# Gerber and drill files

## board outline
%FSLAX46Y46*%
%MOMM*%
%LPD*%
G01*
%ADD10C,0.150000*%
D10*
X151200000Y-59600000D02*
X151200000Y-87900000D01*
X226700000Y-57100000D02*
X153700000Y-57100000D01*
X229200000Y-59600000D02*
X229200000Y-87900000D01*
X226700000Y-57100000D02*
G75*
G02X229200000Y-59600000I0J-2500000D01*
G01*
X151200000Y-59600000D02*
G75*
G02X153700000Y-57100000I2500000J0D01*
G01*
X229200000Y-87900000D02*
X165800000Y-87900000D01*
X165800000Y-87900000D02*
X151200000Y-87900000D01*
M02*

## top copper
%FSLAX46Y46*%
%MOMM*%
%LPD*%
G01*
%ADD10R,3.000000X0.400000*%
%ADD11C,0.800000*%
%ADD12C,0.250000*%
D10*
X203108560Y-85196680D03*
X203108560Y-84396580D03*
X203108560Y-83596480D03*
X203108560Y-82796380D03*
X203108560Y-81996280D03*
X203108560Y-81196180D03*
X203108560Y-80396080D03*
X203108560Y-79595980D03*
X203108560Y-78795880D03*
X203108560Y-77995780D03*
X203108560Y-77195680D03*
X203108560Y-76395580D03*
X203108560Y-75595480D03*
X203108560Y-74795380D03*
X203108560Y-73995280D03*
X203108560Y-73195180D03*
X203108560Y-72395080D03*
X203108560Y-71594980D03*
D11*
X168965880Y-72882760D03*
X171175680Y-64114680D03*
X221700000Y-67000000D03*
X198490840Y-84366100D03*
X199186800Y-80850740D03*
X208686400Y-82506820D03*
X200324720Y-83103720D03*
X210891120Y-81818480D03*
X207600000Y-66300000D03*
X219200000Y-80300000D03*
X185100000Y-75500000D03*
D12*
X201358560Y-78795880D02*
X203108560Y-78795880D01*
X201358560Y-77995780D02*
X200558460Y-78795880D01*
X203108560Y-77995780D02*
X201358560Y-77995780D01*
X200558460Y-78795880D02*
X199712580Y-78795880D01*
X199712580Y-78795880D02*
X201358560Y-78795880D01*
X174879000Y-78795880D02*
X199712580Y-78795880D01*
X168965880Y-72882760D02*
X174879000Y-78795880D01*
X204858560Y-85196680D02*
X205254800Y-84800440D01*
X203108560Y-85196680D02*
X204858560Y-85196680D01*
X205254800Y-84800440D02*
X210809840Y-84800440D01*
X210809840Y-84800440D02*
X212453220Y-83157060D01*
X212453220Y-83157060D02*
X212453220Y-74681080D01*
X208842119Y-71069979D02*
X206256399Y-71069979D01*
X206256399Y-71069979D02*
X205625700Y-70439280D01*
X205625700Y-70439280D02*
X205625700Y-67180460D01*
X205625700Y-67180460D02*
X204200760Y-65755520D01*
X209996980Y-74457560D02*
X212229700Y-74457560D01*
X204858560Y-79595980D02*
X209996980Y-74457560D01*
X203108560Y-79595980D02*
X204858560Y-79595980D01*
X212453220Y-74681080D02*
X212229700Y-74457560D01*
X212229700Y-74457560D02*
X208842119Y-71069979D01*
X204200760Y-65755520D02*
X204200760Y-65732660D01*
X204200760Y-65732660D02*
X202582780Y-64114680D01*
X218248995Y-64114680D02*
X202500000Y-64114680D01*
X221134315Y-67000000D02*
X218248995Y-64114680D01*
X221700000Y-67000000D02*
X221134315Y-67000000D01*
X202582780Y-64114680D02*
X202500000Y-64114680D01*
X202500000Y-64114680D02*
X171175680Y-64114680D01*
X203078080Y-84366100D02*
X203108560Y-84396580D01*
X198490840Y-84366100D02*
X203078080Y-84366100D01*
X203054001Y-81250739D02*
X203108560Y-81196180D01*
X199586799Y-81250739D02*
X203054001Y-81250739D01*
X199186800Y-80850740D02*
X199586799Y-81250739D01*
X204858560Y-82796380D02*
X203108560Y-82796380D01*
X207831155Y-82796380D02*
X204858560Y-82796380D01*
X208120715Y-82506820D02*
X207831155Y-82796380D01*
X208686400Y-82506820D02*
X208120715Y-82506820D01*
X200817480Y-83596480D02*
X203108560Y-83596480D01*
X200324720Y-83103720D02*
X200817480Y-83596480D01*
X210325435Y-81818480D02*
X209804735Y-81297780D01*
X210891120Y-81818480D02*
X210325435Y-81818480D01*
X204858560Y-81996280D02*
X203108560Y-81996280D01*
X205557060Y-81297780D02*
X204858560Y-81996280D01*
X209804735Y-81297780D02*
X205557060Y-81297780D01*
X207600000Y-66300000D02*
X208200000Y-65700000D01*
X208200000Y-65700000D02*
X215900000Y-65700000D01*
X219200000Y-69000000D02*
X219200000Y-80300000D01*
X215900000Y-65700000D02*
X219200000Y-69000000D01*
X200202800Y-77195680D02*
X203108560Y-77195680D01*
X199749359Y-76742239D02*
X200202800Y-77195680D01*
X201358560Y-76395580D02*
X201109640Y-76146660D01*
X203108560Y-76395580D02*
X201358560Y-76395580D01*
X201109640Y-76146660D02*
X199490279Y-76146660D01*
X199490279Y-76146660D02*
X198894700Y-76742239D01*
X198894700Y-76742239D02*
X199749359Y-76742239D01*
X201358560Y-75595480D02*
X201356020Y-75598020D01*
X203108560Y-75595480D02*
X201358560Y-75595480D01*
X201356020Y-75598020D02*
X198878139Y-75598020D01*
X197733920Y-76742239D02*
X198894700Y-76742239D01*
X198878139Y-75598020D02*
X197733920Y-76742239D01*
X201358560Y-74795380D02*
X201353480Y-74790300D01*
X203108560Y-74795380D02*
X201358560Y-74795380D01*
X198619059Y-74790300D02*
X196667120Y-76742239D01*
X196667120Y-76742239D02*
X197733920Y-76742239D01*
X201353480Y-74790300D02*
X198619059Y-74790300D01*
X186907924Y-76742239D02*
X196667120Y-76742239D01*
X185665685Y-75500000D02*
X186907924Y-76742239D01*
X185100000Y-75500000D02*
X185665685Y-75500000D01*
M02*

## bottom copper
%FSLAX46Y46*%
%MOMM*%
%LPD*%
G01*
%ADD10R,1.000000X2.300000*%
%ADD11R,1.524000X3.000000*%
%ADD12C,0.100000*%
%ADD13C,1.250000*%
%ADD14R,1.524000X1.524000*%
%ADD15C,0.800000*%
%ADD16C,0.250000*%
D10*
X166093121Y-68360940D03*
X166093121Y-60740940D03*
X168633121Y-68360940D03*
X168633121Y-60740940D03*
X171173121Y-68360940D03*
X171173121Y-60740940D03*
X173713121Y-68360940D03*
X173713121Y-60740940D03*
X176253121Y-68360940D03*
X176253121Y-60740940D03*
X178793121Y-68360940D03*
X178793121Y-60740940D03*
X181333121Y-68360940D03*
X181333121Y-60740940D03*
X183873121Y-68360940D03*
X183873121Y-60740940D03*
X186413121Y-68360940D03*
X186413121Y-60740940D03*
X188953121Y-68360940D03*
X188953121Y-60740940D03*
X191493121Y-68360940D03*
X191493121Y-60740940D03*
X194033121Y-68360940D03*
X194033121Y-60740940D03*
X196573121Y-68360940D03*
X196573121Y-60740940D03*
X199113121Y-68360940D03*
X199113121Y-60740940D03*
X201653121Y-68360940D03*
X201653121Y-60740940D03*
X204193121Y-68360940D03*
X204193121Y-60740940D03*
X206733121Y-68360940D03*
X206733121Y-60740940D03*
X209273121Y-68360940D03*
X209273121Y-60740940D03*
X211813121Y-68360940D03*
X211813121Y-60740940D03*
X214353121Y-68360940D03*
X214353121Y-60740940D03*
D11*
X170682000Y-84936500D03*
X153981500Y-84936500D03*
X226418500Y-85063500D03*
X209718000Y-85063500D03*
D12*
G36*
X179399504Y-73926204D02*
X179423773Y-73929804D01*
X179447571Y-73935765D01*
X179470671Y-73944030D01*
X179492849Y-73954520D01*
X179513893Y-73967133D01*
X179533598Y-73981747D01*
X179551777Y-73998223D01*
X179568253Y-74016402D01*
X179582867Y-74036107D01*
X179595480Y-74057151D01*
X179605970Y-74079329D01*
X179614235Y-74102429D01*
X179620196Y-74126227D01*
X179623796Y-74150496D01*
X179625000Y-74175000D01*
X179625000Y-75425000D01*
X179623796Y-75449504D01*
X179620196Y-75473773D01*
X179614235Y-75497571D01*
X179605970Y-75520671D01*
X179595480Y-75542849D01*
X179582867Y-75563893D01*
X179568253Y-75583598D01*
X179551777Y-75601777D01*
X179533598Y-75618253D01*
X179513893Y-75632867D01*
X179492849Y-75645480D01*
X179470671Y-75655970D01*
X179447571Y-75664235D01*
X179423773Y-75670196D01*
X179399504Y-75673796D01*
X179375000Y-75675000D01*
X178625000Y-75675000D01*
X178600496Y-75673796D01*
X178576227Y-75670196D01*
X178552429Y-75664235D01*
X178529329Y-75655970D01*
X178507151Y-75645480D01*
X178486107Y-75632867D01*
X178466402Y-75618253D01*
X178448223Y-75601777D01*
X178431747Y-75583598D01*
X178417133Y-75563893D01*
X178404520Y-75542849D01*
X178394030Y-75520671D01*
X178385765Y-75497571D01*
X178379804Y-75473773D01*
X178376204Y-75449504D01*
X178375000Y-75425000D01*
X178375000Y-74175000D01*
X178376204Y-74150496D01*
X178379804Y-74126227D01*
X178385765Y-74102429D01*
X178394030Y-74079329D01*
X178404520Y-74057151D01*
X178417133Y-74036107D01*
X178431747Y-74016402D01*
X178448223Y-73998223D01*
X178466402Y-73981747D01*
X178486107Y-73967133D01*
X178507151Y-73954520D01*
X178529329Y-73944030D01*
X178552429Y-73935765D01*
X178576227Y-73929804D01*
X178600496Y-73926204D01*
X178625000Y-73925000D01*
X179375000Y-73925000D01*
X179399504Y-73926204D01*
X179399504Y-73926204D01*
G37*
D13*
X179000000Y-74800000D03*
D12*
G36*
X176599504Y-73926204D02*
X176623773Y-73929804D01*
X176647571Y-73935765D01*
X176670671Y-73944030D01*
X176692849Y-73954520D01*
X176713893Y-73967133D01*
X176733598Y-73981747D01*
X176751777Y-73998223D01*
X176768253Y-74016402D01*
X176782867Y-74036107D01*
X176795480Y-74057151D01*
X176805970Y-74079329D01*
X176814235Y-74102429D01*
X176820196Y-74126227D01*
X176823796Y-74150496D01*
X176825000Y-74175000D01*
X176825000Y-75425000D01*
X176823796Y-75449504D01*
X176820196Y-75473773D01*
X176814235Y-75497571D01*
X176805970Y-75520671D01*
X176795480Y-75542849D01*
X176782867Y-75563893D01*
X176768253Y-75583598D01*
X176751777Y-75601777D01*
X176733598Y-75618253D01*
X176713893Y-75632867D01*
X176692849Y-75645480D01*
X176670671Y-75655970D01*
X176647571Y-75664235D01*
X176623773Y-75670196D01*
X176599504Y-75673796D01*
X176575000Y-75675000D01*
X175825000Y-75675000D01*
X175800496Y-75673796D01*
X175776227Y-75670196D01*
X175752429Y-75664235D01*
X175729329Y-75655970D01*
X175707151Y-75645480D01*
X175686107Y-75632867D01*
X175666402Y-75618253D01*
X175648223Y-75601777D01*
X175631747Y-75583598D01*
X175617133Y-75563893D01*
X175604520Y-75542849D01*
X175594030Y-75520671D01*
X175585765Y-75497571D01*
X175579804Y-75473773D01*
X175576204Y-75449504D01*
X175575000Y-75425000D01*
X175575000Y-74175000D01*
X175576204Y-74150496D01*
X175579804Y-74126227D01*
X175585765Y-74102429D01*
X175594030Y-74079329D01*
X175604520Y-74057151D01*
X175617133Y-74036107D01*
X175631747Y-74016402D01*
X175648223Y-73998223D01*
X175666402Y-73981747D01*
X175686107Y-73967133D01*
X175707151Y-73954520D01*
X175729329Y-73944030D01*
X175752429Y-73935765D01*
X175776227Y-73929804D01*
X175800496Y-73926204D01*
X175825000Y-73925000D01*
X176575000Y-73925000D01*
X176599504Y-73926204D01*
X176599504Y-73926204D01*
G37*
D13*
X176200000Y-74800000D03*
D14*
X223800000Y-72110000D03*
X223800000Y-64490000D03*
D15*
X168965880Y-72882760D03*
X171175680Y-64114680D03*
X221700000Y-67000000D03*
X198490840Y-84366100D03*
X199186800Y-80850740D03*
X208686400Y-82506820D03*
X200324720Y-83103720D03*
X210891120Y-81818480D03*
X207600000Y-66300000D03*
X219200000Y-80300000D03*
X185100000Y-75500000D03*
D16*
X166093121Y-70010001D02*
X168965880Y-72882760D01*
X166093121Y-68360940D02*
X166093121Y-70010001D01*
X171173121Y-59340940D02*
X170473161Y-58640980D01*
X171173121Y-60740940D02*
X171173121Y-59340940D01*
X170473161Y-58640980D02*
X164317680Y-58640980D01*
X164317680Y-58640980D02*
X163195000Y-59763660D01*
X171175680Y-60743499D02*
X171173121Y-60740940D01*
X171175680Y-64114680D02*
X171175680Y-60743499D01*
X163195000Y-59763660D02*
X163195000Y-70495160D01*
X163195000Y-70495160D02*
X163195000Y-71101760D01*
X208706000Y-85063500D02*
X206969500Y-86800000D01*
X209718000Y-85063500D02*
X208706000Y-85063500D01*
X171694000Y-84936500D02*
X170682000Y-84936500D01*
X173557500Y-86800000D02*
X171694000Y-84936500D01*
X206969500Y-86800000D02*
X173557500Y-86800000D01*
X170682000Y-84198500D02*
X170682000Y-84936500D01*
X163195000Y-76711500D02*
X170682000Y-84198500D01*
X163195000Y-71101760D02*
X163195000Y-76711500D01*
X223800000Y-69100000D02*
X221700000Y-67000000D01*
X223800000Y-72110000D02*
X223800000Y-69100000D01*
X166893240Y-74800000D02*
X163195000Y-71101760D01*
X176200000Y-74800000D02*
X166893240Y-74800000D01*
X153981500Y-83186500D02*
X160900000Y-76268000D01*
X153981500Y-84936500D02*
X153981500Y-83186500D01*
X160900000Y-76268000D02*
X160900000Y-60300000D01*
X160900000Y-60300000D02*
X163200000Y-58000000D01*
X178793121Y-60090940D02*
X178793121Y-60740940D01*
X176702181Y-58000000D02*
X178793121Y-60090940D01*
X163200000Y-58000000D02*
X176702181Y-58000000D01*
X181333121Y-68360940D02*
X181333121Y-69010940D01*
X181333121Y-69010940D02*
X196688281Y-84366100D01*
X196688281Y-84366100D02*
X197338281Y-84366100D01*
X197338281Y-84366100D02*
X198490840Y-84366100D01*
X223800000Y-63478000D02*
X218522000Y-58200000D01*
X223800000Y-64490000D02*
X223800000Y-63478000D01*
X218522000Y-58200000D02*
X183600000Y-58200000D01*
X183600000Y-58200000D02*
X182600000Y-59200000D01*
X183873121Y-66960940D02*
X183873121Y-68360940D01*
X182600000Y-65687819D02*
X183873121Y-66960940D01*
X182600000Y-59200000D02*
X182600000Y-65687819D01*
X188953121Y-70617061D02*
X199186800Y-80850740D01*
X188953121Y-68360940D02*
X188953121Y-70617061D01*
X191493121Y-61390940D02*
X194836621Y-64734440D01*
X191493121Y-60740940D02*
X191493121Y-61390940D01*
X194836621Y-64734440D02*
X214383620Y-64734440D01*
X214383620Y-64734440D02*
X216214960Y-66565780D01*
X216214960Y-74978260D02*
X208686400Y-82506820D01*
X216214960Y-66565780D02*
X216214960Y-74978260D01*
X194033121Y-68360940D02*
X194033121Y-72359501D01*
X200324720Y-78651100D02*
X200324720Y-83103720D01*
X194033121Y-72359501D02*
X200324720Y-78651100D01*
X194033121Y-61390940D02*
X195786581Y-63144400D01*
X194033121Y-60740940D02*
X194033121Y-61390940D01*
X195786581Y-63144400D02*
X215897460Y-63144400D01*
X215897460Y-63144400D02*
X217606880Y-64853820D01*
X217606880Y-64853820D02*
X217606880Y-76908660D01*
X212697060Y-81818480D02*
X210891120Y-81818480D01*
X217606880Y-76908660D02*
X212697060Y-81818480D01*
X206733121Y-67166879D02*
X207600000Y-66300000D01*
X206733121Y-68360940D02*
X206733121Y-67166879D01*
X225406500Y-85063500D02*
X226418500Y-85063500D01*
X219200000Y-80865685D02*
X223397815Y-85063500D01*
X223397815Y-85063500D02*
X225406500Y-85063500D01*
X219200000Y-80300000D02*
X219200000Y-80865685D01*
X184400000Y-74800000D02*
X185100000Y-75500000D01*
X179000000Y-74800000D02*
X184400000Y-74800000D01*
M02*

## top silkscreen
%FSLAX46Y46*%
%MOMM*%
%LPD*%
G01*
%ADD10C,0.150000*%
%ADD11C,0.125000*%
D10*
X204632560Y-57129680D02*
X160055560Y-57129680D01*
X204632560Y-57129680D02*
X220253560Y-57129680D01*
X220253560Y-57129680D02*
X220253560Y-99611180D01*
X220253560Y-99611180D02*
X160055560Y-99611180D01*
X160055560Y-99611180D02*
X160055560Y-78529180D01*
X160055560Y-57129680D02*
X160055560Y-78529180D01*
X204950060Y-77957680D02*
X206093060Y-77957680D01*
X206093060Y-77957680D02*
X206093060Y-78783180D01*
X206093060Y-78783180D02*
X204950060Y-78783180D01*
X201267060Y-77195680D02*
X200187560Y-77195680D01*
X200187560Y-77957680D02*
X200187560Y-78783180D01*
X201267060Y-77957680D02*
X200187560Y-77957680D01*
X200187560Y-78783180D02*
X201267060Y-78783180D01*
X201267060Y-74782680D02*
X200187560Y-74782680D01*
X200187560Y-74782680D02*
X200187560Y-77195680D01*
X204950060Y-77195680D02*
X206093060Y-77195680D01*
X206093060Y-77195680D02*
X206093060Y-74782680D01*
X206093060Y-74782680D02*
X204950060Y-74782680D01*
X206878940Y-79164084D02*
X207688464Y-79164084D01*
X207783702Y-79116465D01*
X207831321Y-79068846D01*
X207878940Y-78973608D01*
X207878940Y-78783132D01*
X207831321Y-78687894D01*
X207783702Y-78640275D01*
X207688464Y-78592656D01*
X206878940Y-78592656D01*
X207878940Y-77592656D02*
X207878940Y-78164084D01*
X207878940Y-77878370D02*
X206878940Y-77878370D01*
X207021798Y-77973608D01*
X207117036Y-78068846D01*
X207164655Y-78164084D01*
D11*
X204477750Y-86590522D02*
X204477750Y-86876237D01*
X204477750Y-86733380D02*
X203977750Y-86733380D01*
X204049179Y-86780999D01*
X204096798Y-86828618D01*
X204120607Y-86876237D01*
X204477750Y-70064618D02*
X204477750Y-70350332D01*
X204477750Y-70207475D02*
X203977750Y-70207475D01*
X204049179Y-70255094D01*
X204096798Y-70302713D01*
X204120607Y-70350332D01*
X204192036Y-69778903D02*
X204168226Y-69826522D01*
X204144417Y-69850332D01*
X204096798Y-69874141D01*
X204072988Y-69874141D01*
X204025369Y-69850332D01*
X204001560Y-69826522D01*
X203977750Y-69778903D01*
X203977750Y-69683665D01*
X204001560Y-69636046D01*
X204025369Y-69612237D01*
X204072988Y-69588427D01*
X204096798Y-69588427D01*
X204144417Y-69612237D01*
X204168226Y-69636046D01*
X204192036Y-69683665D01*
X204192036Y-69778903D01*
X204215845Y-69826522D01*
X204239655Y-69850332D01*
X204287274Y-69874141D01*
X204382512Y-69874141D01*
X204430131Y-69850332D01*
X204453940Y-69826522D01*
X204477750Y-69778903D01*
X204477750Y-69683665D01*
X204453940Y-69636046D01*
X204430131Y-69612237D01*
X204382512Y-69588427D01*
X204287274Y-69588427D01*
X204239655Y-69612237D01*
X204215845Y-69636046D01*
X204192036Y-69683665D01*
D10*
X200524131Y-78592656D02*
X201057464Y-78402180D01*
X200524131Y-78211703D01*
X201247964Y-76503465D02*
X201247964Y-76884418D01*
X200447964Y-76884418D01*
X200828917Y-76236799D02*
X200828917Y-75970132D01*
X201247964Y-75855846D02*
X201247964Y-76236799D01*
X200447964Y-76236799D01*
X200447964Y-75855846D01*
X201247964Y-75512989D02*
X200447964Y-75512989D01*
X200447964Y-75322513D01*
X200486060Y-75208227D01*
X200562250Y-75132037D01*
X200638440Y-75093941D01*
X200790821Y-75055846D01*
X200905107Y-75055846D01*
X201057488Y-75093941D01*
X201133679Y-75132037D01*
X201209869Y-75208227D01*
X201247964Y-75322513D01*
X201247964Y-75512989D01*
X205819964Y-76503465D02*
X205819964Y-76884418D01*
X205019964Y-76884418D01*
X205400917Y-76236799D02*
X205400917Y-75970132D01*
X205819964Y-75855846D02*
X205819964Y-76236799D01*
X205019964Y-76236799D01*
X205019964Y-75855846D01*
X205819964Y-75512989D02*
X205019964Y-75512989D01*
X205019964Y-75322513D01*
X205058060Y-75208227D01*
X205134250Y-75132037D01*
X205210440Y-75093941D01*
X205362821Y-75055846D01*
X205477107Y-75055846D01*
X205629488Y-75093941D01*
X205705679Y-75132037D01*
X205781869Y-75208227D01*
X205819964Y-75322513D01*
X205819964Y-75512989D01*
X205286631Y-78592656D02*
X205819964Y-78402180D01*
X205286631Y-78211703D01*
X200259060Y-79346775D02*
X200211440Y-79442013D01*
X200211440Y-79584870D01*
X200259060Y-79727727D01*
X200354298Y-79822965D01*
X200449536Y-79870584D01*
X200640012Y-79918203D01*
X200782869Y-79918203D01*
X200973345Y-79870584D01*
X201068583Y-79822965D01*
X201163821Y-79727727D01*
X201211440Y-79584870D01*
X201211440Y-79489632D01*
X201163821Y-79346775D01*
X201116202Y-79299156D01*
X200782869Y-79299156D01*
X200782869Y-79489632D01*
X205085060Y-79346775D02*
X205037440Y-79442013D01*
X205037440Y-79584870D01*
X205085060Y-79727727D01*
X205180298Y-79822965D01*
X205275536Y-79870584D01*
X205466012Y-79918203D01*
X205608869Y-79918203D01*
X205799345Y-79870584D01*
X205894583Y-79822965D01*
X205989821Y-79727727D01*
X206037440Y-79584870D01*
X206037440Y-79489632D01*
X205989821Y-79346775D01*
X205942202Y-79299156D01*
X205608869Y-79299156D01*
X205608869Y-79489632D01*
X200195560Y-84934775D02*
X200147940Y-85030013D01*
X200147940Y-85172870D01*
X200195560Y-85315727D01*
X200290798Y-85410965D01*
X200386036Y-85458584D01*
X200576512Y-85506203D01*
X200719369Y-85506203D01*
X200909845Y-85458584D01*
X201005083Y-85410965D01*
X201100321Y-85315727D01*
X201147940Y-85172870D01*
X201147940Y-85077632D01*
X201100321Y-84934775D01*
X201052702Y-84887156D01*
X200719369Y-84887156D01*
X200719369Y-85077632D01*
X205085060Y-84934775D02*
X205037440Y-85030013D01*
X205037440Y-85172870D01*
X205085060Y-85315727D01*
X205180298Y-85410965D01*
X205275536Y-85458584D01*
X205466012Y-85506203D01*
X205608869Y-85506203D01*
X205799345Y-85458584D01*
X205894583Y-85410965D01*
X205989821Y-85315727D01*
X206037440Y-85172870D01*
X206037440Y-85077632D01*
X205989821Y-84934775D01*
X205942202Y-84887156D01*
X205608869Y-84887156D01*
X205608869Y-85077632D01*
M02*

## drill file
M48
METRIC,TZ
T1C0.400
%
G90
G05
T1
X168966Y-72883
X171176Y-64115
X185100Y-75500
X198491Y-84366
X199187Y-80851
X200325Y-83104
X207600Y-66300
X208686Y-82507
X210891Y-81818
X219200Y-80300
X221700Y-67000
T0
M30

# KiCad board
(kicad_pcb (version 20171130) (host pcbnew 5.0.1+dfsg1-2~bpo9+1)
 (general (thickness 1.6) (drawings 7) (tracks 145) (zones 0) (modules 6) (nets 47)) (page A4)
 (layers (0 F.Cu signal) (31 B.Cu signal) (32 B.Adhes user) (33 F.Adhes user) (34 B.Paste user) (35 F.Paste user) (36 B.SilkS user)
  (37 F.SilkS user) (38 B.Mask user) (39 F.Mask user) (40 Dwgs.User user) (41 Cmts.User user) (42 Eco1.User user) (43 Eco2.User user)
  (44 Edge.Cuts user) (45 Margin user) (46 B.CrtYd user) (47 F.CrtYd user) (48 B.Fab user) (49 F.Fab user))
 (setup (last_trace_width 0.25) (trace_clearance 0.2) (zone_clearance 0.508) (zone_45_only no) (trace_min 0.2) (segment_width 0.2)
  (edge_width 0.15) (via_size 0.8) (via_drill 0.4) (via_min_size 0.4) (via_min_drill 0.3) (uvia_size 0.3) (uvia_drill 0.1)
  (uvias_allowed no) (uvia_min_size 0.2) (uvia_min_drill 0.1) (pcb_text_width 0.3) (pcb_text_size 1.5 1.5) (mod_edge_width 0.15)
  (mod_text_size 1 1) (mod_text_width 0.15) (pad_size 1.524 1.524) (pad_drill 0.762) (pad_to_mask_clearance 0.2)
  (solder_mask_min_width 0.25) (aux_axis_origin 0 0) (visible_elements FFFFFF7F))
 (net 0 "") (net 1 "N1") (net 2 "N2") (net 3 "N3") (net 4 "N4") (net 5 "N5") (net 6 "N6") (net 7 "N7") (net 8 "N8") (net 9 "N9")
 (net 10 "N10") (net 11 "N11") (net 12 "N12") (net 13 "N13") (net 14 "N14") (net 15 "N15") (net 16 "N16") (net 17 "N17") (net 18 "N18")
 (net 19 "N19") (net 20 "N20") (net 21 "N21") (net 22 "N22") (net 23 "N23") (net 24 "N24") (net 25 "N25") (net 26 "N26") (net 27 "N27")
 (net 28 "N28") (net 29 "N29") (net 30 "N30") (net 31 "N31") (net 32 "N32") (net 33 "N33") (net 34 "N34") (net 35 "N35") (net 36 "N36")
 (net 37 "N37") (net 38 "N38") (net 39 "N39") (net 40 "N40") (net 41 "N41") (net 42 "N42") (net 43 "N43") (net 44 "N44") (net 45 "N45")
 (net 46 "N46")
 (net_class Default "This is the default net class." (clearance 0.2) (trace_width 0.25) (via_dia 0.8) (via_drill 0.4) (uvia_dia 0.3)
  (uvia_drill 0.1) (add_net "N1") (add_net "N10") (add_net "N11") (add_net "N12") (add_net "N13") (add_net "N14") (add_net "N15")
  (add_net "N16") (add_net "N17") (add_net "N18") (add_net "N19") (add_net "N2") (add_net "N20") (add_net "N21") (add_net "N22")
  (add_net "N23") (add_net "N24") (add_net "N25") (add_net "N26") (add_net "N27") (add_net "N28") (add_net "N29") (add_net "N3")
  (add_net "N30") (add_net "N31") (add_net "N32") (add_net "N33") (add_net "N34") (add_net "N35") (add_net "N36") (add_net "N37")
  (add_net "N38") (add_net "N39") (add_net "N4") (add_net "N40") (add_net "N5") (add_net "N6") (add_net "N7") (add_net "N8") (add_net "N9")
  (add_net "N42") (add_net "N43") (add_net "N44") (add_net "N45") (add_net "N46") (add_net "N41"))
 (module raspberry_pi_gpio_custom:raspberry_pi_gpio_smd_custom (layer B.Cu) (at 190.223121 64.55094)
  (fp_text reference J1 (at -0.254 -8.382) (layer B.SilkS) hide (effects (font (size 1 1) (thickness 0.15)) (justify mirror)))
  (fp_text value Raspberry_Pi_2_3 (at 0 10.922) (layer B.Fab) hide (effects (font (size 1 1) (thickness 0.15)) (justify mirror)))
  (pad 1 smd rect (at -24.13 3.81) (size 1 2.3) (layers B.Cu B.Paste B.Mask) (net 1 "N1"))
  (pad 2 smd rect (at -24.13 -3.81) (size 1 2.3) (layers B.Cu B.Paste B.Mask) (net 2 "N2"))
  (pad 3 smd rect (at -21.59 3.81) (size 1 2.3) (layers B.Cu B.Paste B.Mask) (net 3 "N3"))
  (pad 4 smd rect (at -21.59 -3.81) (size 1 2.3) (layers B.Cu B.Paste B.Mask) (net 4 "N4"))
  (pad 5 smd rect (at -19.05 3.81) (size 1 2.3) (layers B.Cu B.Paste B.Mask) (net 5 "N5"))
  (pad 6 smd rect (at -19.05 -3.81) (size 1 2.3) (layers B.Cu B.Paste B.Mask) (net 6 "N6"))
  (pad 7 smd rect (at -16.51 3.81) (size 1 2.3) (layers B.Cu B.Paste B.Mask) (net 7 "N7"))
  (pad 8 smd rect (at -16.51 -3.81) (size 1 2.3) (layers B.Cu B.Paste B.Mask) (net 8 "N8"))
  (pad 9 smd rect (at -13.97 3.81) (size 1 2.3) (layers B.Cu B.Paste B.Mask) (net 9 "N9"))
  (pad 10 smd rect (at -13.97 -3.81) (size 1 2.3) (layers B.Cu B.Paste B.Mask) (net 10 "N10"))
  (pad 11 smd rect (at -11.43 3.81) (size 1 2.3) (layers B.Cu B.Paste B.Mask) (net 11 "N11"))
  (pad 12 smd rect (at -11.43 -3.81) (size 1 2.3) (layers B.Cu B.Paste B.Mask) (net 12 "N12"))
  (pad 13 smd rect (at -8.89 3.81) (size 1 2.3) (layers B.Cu B.Paste B.Mask) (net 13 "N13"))
  (pad 14 smd rect (at -8.89 -3.81) (size 1 2.3) (layers B.Cu B.Paste B.Mask) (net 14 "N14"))
  (pad 15 smd rect (at -6.35 3.81) (size 1 2.3) (layers B.Cu B.Paste B.Mask) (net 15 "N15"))
  (pad 16 smd rect (at -6.35 -3.81) (size 1 2.3) (layers B.Cu B.Paste B.Mask) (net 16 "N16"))
  (pad 17 smd rect (at -3.81 3.81) (size 1 2.3) (layers B.Cu B.Paste B.Mask) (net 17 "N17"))
  (pad 18 smd rect (at -3.81 -3.81) (size 1 2.3) (layers B.Cu B.Paste B.Mask) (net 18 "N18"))
  (pad 19 smd rect (at -1.27 3.81) (size 1 2.3) (layers B.Cu B.Paste B.Mask) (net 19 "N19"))
  (pad 20 smd rect (at -1.27 -3.81) (size 1 2.3) (layers B.Cu B.Paste B.Mask) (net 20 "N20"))
  (pad 21 smd rect (at 1.27 3.81) (size 1 2.3) (layers B.Cu B.Paste B.Mask) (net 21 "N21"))
  (pad 22 smd rect (at 1.27 -3.81) (size 1 2.3) (layers B.Cu B.Paste B.Mask) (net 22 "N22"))
  (pad 23 smd rect (at 3.81 3.81) (size 1 2.3) (layers B.Cu B.Paste B.Mask) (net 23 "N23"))
  (pad 24 smd rect (at 3.81 -3.81) (size 1 2.3) (layers B.Cu B.Paste B.Mask) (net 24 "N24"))
  (pad 25 smd rect (at 6.35 3.81) (size 1 2.3) (layers B.Cu B.Paste B.Mask) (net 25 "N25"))
  (pad 26 smd rect (at 6.35 -3.81) (size 1 2.3) (layers B.Cu B.Paste B.Mask) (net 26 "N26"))
  (pad 27 smd rect (at 8.89 3.81) (size 1 2.3) (layers B.Cu B.Paste B.Mask) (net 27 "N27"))
  (pad 28 smd rect (at 8.89 -3.81) (size 1 2.3) (layers B.Cu B.Paste B.Mask) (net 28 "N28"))
  (pad 29 smd rect (at 11.43 3.81) (size 1 2.3) (layers B.Cu B.Paste B.Mask) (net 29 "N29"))
  (pad 30 smd rect (at 11.43 -3.81) (size 1 2.3) (layers B.Cu B.Paste B.Mask) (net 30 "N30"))
  (pad 31 smd rect (at 13.97 3.81) (size 1 2.3) (layers B.Cu B.Paste B.Mask) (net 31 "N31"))
  (pad 32 smd rect (at 13.97 -3.81) (size 1 2.3) (layers B.Cu B.Paste B.Mask) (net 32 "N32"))
  (pad 33 smd rect (at 16.51 3.81) (size 1 2.3) (layers B.Cu B.Paste B.Mask) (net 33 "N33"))
  (pad 34 smd rect (at 16.51 -3.81) (size 1 2.3) (layers B.Cu B.Paste B.Mask) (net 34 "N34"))
  (pad 35 smd rect (at 19.05 3.81) (size 1 2.3) (layers B.Cu B.Paste B.Mask) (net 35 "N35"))
  (pad 36 smd rect (at 19.05 -3.81) (size 1 2.3) (layers B.Cu B.Paste B.Mask) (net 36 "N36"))
  (pad 37 smd rect (at 21.59 3.81) (size 1 2.3) (layers B.Cu B.Paste B.Mask) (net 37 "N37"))
  (pad 38 smd rect (at 21.59 -3.81) (size 1 2.3) (layers B.Cu B.Paste B.Mask) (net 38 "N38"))
  (pad 39 smd rect (at 24.13 3.81) (size 1 2.3) (layers B.Cu B.Paste B.Mask) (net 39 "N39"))
  (pad 40 smd rect (at 24.13 -3.81) (size 1 2.3) (layers B.Cu B.Paste B.Mask) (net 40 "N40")))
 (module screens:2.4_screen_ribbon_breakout (layer F.Cu) (at 204.63256 78.40218 90)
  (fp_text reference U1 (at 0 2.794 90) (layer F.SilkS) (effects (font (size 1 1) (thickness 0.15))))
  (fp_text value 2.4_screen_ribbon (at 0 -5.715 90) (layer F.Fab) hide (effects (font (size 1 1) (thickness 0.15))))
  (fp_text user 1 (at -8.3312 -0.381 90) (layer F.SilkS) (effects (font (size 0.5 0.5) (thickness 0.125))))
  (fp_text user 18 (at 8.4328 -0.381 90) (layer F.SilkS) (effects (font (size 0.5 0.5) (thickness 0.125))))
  (fp_line (start 21.2725 0) (end 21.2725 -44.577) (layer F.SilkS) (width 0.15))
  (fp_line (start 21.2725 0) (end 21.2725 15.621) (layer F.SilkS) (width 0.15))
  (fp_line (start 21.2725 15.621) (end -21.209 15.621) (layer F.SilkS) (width 0.15))
  (fp_line (start -21.209 15.621) (end -21.209 -44.577) (layer F.SilkS) (width 0.15))
  (fp_line (start -21.209 -44.577) (end -0.127 -44.577) (layer F.SilkS) (width 0.15))
  (fp_line (start 21.2725 -44.577) (end -0.127 -44.577) (layer F.SilkS) (width 0.15))
  (fp_line (start 0.4445 0.3175) (end 0.4445 1.4605) (layer F.SilkS) (width 0.15))
  (fp_line (start 0.4445 1.4605) (end -0.381 1.4605) (layer F.SilkS) (width 0.15))
  (fp_line (start -0.381 1.4605) (end -0.381 0.3175) (layer F.SilkS) (width 0.15))
  (fp_line (start 1.2065 -3.3655) (end 1.2065 -4.445) (layer F.SilkS) (width 0.15))
  (fp_line (start 0.4445 -4.445) (end -0.381 -4.445) (layer F.SilkS) (width 0.15))
  (fp_line (start 0.4445 -3.3655) (end 0.4445 -4.445) (layer F.SilkS) (width 0.15))
  (fp_line (start -0.381 -4.445) (end -0.381 -3.3655) (layer F.SilkS) (width 0.15))
  (fp_line (start 3.6195 -3.3655) (end 3.6195 -4.445) (layer F.SilkS) (width 0.15))
  (fp_line (start 3.6195 -4.445) (end 1.2065 -4.445) (layer F.SilkS) (width 0.15))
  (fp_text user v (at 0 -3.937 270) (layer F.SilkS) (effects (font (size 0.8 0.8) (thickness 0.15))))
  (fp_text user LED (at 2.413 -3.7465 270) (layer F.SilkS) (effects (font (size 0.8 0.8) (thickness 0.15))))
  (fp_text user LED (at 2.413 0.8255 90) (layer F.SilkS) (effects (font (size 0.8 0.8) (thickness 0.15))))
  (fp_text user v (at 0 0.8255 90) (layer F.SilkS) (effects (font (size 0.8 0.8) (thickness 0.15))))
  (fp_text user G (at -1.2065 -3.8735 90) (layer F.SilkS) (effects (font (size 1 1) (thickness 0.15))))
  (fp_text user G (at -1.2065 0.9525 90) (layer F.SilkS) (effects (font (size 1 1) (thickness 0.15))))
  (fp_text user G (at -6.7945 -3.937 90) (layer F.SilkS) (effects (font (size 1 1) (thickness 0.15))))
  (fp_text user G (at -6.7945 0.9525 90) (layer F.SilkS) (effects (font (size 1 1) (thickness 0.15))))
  (fp_line (start 1.2065 0.3175) (end 1.2065 1.4605) (layer F.SilkS) (width 0.15))
  (fp_line (start 1.2065 1.4605) (end 3.6195 1.4605) (layer F.SilkS) (width 0.15))
  (fp_line (start 3.6195 1.4605) (end 3.6195 0.3175) (layer F.SilkS) (width 0.15))
  (pad 1 smd rect (at -6.7945 -1.524 90) (size 0.4 3) (layers F.Cu F.Paste F.Mask) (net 6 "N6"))
  (pad 2 smd rect (at -5.9944 -1.524 90) (size 0.4 3) (layers F.Cu F.Paste F.Mask) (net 13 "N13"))
  (pad 3 smd rect (at -5.1943 -1.524 90) (size 0.4 3) (layers F.Cu F.Paste F.Mask) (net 23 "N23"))
  (pad 4 smd rect (at -4.3942 -1.524 90) (size 0.4 3) (layers F.Cu F.Paste F.Mask) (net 22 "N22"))
  (pad 5 smd rect (at -3.5941 -1.524 90) (size 0.4 3) (layers F.Cu F.Paste F.Mask) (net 24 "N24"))
  (pad 6 smd rect (at -2.794 -1.524 90) (size 0.4 3) (layers F.Cu F.Paste F.Mask) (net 19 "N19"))
  (pad 7 smd rect (at -1.9939 -1.524 90) (size 0.4 3) (layers F.Cu F.Paste F.Mask) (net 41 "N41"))
  (pad 8 smd rect (at -1.1938 -1.524 90) (size 0.4 3) (layers F.Cu F.Paste F.Mask) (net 6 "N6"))
  (pad 9 smd rect (at -0.3937 -1.524 90) (size 0.4 3) (layers F.Cu F.Paste F.Mask) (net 1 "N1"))
  (pad 10 smd rect (at 0.4064 -1.524 90) (size 0.4 3) (layers F.Cu F.Paste F.Mask) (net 1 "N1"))
  (pad 11 smd rect (at 1.2065 -1.524 90) (size 0.4 3) (layers F.Cu F.Paste F.Mask) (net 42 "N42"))
  (pad 12 smd rect (at 2.0066 -1.524 90) (size 0.4 3) (layers F.Cu F.Paste F.Mask) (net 42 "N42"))
  (pad 13 smd rect (at 2.8067 -1.524 90) (size 0.4 3) (layers F.Cu F.Paste F.Mask) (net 42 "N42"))
  (pad 14 smd rect (at 3.6068 -1.524 90) (size 0.4 3) (layers F.Cu F.Paste F.Mask) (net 42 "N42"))
  (pad 15 smd rect (at 4.4069 -1.524 90) (size 0.4 3) (layers F.Cu F.Paste F.Mask) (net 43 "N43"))
  (pad 16 smd rect (at 5.207 -1.524 90) (size 0.4 3) (layers F.Cu F.Paste F.Mask) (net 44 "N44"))
  (pad 17 smd rect (at 6.0071 -1.524 90) (size 0.4 3) (layers F.Cu F.Paste F.Mask) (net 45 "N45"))
  (pad 18 smd rect (at 6.8072 -1.524 90) (size 0.4 3) (layers F.Cu F.Paste F.Mask) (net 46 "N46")))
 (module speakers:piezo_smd (layer B.Cu) (at 162.3 85 180)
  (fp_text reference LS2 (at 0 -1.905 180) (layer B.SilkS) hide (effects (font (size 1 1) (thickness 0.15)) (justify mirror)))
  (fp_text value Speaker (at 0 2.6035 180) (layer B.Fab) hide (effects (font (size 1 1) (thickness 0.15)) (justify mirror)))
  (pad 2 smd rect (at -8.382 0.0635 180) (size 1.524 3) (layers B.Cu B.Paste B.Mask) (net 6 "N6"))
  (pad 1 smd rect (at 8.3185 0.0635 180) (size 1.524 3) (layers B.Cu B.Paste B.Mask) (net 12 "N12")))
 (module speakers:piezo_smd (layer B.Cu) (at 218.1 85)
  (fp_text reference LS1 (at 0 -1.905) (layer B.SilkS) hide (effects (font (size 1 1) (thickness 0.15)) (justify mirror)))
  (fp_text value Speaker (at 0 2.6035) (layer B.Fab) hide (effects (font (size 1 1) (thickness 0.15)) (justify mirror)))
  (pad 1 smd rect (at 8.3185 0.0635) (size 1.524 3) (layers B.Cu B.Paste B.Mask) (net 33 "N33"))
  (pad 2 smd rect (at -8.382 0.0635) (size 1.524 3) (layers B.Cu B.Paste B.Mask) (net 6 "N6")))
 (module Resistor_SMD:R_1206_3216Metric (layer B.Cu) (at 177.6 74.8 180)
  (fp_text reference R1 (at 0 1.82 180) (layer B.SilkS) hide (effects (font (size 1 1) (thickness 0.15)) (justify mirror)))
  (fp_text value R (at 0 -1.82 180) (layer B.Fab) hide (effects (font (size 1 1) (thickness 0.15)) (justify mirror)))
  (pad 1 smd roundrect (at -1.4 0 180) (size 1.25 1.75) (layers B.Cu B.Paste B.Mask) (roundrect_rratio 0.2) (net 42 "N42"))
  (pad 2 smd roundrect (at 1.4 0 180) (size 1.25 1.75) (layers B.Cu B.Paste B.Mask) (roundrect_rratio 0.2) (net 6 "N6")))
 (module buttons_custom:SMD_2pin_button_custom (layer B.Cu) (at 223.8 68.3 270)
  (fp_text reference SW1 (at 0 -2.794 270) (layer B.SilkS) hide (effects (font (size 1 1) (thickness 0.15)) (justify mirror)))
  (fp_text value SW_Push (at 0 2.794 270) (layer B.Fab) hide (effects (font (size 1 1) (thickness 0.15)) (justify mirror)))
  (pad 1 smd rect (at 3.81 0 270) (size 1.524 1.524) (layers B.Cu B.Paste B.Mask) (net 6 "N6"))
  (pad 2 smd rect (at -3.81 0 270) (size 1.524 1.524) (layers B.Cu B.Paste B.Mask) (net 15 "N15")))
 (gr_line (start 151.2 59.6) (end 151.2 87.9) (layer Edge.Cuts) (width 0.15))
 (gr_line (start 226.7 57.1) (end 153.7 57.1) (layer Edge.Cuts) (width 0.15))
 (gr_line (start 229.2 59.6) (end 229.2 87.9) (layer Edge.Cuts) (width 0.15))
 (gr_arc (start 226.7 59.6) (end 229.2 59.6) (angle -90) (layer Edge.Cuts) (width 0.15))
 (gr_arc (start 153.7 59.6) (end 153.7 57.1) (angle -90) (layer Edge.Cuts) (width 0.15))
 (gr_line (start 229.2 87.9) (end 165.8 87.9) (layer Edge.Cuts) (width 0.15))
 (gr_line (start 165.8 87.9) (end 151.2 87.9) (layer Edge.Cuts) (width 0.15))
 (segment (start 201.35856 78.79588) (end 203.10856 78.79588) (width 0.25) (layer F.Cu) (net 1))
 (segment (start 201.35856 77.99578) (end 200.55846 78.79588) (width 0.25) (layer F.Cu) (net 1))
 (segment (start 203.10856 77.99578) (end 201.35856 77.99578) (width 0.25) (layer F.Cu) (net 1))
 (segment (start 200.55846 78.79588) (end 199.71258 78.79588) (width 0.25) (layer F.Cu) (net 1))
 (segment (start 199.71258 78.79588) (end 201.35856 78.79588) (width 0.25) (layer F.Cu) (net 1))
 (via (at 168.96588 72.88276) (size 0.8) (drill 0.4) (layers F.Cu B.Cu) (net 1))
 (segment (start 166.093121 70.010001) (end 168.96588 72.88276) (width 0.25) (layer B.Cu) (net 1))
 (segment (start 166.093121 68.36094) (end 166.093121 70.010001) (width 0.25) (layer B.Cu) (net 1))
 (segment (start 174.879 78.79588) (end 199.71258 78.79588) (width 0.25) (layer F.Cu) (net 1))
 (segment (start 168.96588 72.88276) (end 174.879 78.79588) (width 0.25) (layer F.Cu) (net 1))
 (segment (start 171.173121 59.34094) (end 170.473161 58.64098) (width 0.25) (layer B.Cu) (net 6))
 (segment (start 171.173121 60.74094) (end 171.173121 59.34094) (width 0.25) (layer B.Cu) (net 6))
 (segment (start 170.473161 58.64098) (end 164.31768 58.64098) (width 0.25) (layer B.Cu) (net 6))
 (segment (start 164.31768 58.64098) (end 163.195 59.76366) (width 0.25) (layer B.Cu) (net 6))
 (segment (start 204.85856 85.19668) (end 205.2548 84.80044) (width 0.25) (layer F.Cu) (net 6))
 (segment (start 203.10856 85.19668) (end 204.85856 85.19668) (width 0.25) (layer F.Cu) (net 6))
 (segment (start 205.2548 84.80044) (end 210.80984 84.80044) (width 0.25) (layer F.Cu) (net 6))
 (segment (start 210.80984 84.80044) (end 212.45322 83.15706) (width 0.25) (layer F.Cu) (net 6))
 (segment (start 212.45322 83.15706) (end 212.45322 74.68108) (width 0.25) (layer F.Cu) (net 6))
 (segment (start 208.842119 71.069979) (end 206.256399 71.069979) (width 0.25) (layer F.Cu) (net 6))
 (segment (start 206.256399 71.069979) (end 205.6257 70.43928) (width 0.25) (layer F.Cu) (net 6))
 (segment (start 205.6257 70.43928) (end 205.6257 67.18046) (width 0.25) (layer F.Cu) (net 6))
 (segment (start 205.6257 67.18046) (end 204.20076 65.75552) (width 0.25) (layer F.Cu) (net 6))
 (via (at 171.17568 64.11468) (size 0.8) (drill 0.4) (layers F.Cu B.Cu) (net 6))
 (segment (start 171.17568 60.743499) (end 171.173121 60.74094) (width 0.25) (layer B.Cu) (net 6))
 (segment (start 171.17568 64.11468) (end 171.17568 60.743499) (width 0.25) (layer B.Cu) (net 6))
 (segment (start 209.99698 74.45756) (end 212.2297 74.45756) (width 0.25) (layer F.Cu) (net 6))
 (segment (start 204.85856 79.59598) (end 209.99698 74.45756) (width 0.25) (layer F.Cu) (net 6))
 (segment (start 203.10856 79.59598) (end 204.85856 79.59598) (width 0.25) (layer F.Cu) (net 6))
 (segment (start 212.45322 74.68108) (end 212.2297 74.45756) (width 0.25) (layer F.Cu) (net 6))
 (segment (start 212.2297 74.45756) (end 208.842119 71.069979) (width 0.25) (layer F.Cu) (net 6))
 (segment (start 204.20076 65.75552) (end 204.20076 65.73266) (width 0.25) (layer F.Cu) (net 6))
 (segment (start 204.20076 65.73266) (end 202.58278 64.11468) (width 0.25) (layer F.Cu) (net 6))
 (segment (start 163.195 59.76366) (end 163.195 70.49516) (width 0.25) (layer B.Cu) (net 6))
 (segment (start 163.195 70.49516) (end 163.195 71.10176) (width 0.25) (layer B.Cu) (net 6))
 (segment (start 208.706 85.0635) (end 206.9695 86.8) (width 0.25) (layer B.Cu) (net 6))
 (segment (start 209.718 85.0635) (end 208.706 85.0635) (width 0.25) (layer B.Cu) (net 6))
 (segment (start 171.694 84.9365) (end 170.682 84.9365) (width 0.25) (layer B.Cu) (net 6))
 (segment (start 173.5575 86.8) (end 171.694 84.9365) (width 0.25) (layer B.Cu) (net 6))
 (segment (start 206.9695 86.8) (end 173.5575 86.8) (width 0.25) (layer B.Cu) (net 6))
 (segment (start 170.682 84.1985) (end 170.682 84.9365) (width 0.25) (layer B.Cu) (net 6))
 (segment (start 163.195 76.7115) (end 170.682 84.1985) (width 0.25) (layer B.Cu) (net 6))
 (segment (start 163.195 71.10176) (end 163.195 76.7115) (width 0.25) (layer B.Cu) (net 6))
 (via (at 221.7 67) (size 0.8) (drill 0.4) (layers F.Cu B.Cu) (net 6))
 (segment (start 223.8 69.1) (end 221.7 67) (width 0.25) (layer B.Cu) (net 6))
 (segment (start 223.8 72.11) (end 223.8 69.1) (width 0.25) (layer B.Cu) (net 6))
 (segment (start 218.248995 64.11468) (end 202.5 64.11468) (width 0.25) (layer F.Cu) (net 6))
 (segment (start 221.134315 67) (end 218.248995 64.11468) (width 0.25) (layer F.Cu) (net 6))
 (segment (start 221.7 67) (end 221.134315 67) (width 0.25) (layer F.Cu) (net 6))
 (segment (start 202.58278 64.11468) (end 202.5 64.11468) (width 0.25) (layer F.Cu) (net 6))
 (segment (start 202.5 64.11468) (end 171.17568 64.11468) (width 0.25) (layer F.Cu) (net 6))
 (segment (start 166.89324 74.8) (end 163.195 71.10176) (width 0.25) (layer B.Cu) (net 6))
 (segment (start 176.2 74.8) (end 166.89324 74.8) (width 0.25) (layer B.Cu) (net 6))
 (segment (start 153.9815 83.1865) (end 160.9 76.268) (width 0.25) (layer B.Cu) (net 12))
 (segment (start 153.9815 84.9365) (end 153.9815 83.1865) (width 0.25) (layer B.Cu) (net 12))
 (segment (start 160.9 76.268) (end 160.9 60.3) (width 0.25) (layer B.Cu) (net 12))
 (segment (start 160.9 60.3) (end 163.2 58) (width 0.25) (layer B.Cu) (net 12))
 (segment (start 178.793121 60.09094) (end 178.793121 60.74094) (width 0.25) (layer B.Cu) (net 12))
 (segment (start 176.702181 58) (end 178.793121 60.09094) (width 0.25) (layer B.Cu) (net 12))
 (segment (start 163.2 58) (end 176.702181 58) (width 0.25) (layer B.Cu) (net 12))
 (via (at 198.49084 84.3661) (size 0.8) (drill 0.4) (layers F.Cu B.Cu) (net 13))
 (segment (start 181.333121 68.36094) (end 181.333121 69.01094) (width 0.25) (layer B.Cu) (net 13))
 (segment (start 181.333121 69.01094) (end 196.688281 84.3661) (width 0.25) (layer B.Cu) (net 13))
 (segment (start 196.688281 84.3661) (end 197.338281 84.3661) (width 0.25) (layer B.Cu) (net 13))
 (segment (start 197.338281 84.3661) (end 198.49084 84.3661) (width 0.25) (layer B.Cu) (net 13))
 (segment (start 203.07808 84.3661) (end 203.10856 84.39658) (width 0.25) (layer F.Cu) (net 13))
 (segment (start 198.49084 84.3661) (end 203.07808 84.3661) (width 0.25) (layer F.Cu) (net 13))
 (segment (start 223.8 63.478) (end 218.522 58.2) (width 0.25) (layer B.Cu) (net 15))
 (segment (start 223.8 64.49) (end 223.8 63.478) (width 0.25) (layer B.Cu) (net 15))
 (segment (start 218.522 58.2) (end 183.6 58.2) (width 0.25) (layer B.Cu) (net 15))
 (segment (start 183.6 58.2) (end 182.6 59.2) (width 0.25) (layer B.Cu) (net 15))
 (segment (start 183.873121 66.96094) (end 183.873121 68.36094) (width 0.25) (layer B.Cu) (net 15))
 (segment (start 182.6 65.687819) (end 183.873121 66.96094) (width 0.25) (layer B.Cu) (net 15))
 (segment (start 182.6 59.2) (end 182.6 65.687819) (width 0.25) (layer B.Cu) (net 15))
 (via (at 199.1868 80.85074) (size 0.8) (drill 0.4) (layers F.Cu B.Cu) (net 19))
 (segment (start 188.953121 70.617061) (end 199.1868 80.85074) (width 0.25) (layer B.Cu) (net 19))
 (segment (start 188.953121 68.36094) (end 188.953121 70.617061) (width 0.25) (layer B.Cu) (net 19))
 (segment (start 203.054001 81.250739) (end 203.10856 81.19618) (width 0.25) (layer F.Cu) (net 19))
 (segment (start 199.586799 81.250739) (end 203.054001 81.250739) (width 0.25) (layer F.Cu) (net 19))
 (segment (start 199.1868 80.85074) (end 199.586799 81.250739) (width 0.25) (layer F.Cu) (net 19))
 (segment (start 191.493121 61.39094) (end 194.836621 64.73444) (width 0.25) (layer B.Cu) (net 22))
 (segment (start 191.493121 60.74094) (end 191.493121 61.39094) (width 0.25) (layer B.Cu) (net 22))
 (segment (start 194.836621 64.73444) (end 214.38362 64.73444) (width 0.25) (layer B.Cu) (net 22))
 (segment (start 214.38362 64.73444) (end 216.21496 66.56578) (width 0.25) (layer B.Cu) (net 22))
 (via (at 208.6864 82.50682) (size 0.8) (drill 0.4) (layers F.Cu B.Cu) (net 22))
 (segment (start 216.21496 74.97826) (end 208.6864 82.50682) (width 0.25) (layer B.Cu) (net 22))
 (segment (start 216.21496 66.56578) (end 216.21496 74.97826) (width 0.25) (layer B.Cu) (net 22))
 (segment (start 204.85856 82.79638) (end 203.10856 82.79638) (width 0.25) (layer F.Cu) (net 22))
 (segment (start 207.831155 82.79638) (end 204.85856 82.79638) (width 0.25) (layer F.Cu) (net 22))
 (segment (start 208.120715 82.50682) (end 207.831155 82.79638) (width 0.25) (layer F.Cu) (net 22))
 (segment (start 208.6864 82.50682) (end 208.120715 82.50682) (width 0.25) (layer F.Cu) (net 22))
 (segment (start 194.033121 68.36094) (end 194.033121 72.359501) (width 0.25) (layer B.Cu) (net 23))
 (via (at 200.32472 83.10372) (size 0.8) (drill 0.4) (layers F.Cu B.Cu) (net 23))
 (segment (start 200.32472 78.6511) (end 200.32472 83.10372) (width 0.25) (layer B.Cu) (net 23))
 (segment (start 194.033121 72.359501) (end 200.32472 78.6511) (width 0.25) (layer B.Cu) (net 23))
 (segment (start 200.81748 83.59648) (end 203.10856 83.59648) (width 0.25) (layer F.Cu) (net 23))
 (segment (start 200.32472 83.10372) (end 200.81748 83.59648) (width 0.25) (layer F.Cu) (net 23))
 (segment (start 194.033121 61.39094) (end 195.786581 63.1444) (width 0.25) (layer B.Cu) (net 24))
 (segment (start 194.033121 60.74094) (end 194.033121 61.39094) (width 0.25) (layer B.Cu) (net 24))
 (segment (start 195.786581 63.1444) (end 215.89746 63.1444) (width 0.25) (layer B.Cu) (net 24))
 (segment (start 215.89746 63.1444) (end 217.60688 64.85382) (width 0.25) (layer B.Cu) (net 24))
 (segment (start 217.60688 64.85382) (end 217.60688 76.90866) (width 0.25) (layer B.Cu) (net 24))
 (via (at 210.89112 81.81848) (size 0.8) (drill 0.4) (layers F.Cu B.Cu) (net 24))
 (segment (start 212.69706 81.81848) (end 210.89112 81.81848) (width 0.25) (layer B.Cu) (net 24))
 (segment (start 217.60688 76.90866) (end 212.69706 81.81848) (width 0.25) (layer B.Cu) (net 24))
 (segment (start 210.325435 81.81848) (end 209.804735 81.29778) (width 0.25) (layer F.Cu) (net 24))
 (segment (start 210.89112 81.81848) (end 210.325435 81.81848) (width 0.25) (layer F.Cu) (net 24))
 (segment (start 204.85856 81.99628) (end 203.10856 81.99628) (width 0.25) (layer F.Cu) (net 24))
 (segment (start 205.55706 81.29778) (end 204.85856 81.99628) (width 0.25) (layer F.Cu) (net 24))
 (segment (start 209.804735 81.29778) (end 205.55706 81.29778) (width 0.25) (layer F.Cu) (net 24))
 (via (at 207.6 66.3) (size 0.8) (drill 0.4) (layers F.Cu B.Cu) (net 33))
 (segment (start 206.733121 67.166879) (end 207.6 66.3) (width 0.25) (layer B.Cu) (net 33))
 (segment (start 206.733121 68.36094) (end 206.733121 67.166879) (width 0.25) (layer B.Cu) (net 33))
 (segment (start 207.6 66.3) (end 208.2 65.7) (width 0.25) (layer F.Cu) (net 33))
 (segment (start 208.2 65.7) (end 215.9 65.7) (width 0.25) (layer F.Cu) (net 33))
 (via (at 219.2 80.3) (size 0.8) (drill 0.4) (layers F.Cu B.Cu) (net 33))
 (segment (start 219.2 69) (end 219.2 80.3) (width 0.25) (layer F.Cu) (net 33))
 (segment (start 215.9 65.7) (end 219.2 69) (width 0.25) (layer F.Cu) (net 33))
 (segment (start 225.4065 85.0635) (end 226.4185 85.0635) (width 0.25) (layer B.Cu) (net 33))
 (segment (start 219.2 80.865685) (end 223.397815 85.0635) (width 0.25) (layer B.Cu) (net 33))
 (segment (start 223.397815 85.0635) (end 225.4065 85.0635) (width 0.25) (layer B.Cu) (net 33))
 (segment (start 219.2 80.3) (end 219.2 80.865685) (width 0.25) (layer B.Cu) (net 33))
 (segment (start 200.2028 77.19568) (end 203.10856 77.19568) (width 0.25) (layer F.Cu) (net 42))
 (segment (start 199.749359 76.742239) (end 200.2028 77.19568) (width 0.25) (layer F.Cu) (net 42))
 (segment (start 201.35856 76.39558) (end 201.10964 76.14666) (width 0.25) (layer F.Cu) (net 42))
 (segment (start 203.10856 76.39558) (end 201.35856 76.39558) (width 0.25) (layer F.Cu) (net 42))
 (segment (start 201.10964 76.14666) (end 199.490279 76.14666) (width 0.25) (layer F.Cu) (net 42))
 (segment (start 199.490279 76.14666) (end 198.8947 76.742239) (width 0.25) (layer F.Cu) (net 42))
 (segment (start 198.8947 76.742239) (end 199.749359 76.742239) (width 0.25) (layer F.Cu) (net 42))
 (segment (start 201.35856 75.59548) (end 201.35602 75.59802) (width 0.25) (layer F.Cu) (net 42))
 (segment (start 203.10856 75.59548) (end 201.35856 75.59548) (width 0.25) (layer F.Cu) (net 42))
 (segment (start 201.35602 75.59802) (end 198.878139 75.59802) (width 0.25) (layer F.Cu) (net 42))
 (segment (start 197.73392 76.742239) (end 198.8947 76.742239) (width 0.25) (layer F.Cu) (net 42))
 (segment (start 198.878139 75.59802) (end 197.73392 76.742239) (width 0.25) (layer F.Cu) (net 42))
 (segment (start 201.35856 74.79538) (end 201.35348 74.7903) (width 0.25) (layer F.Cu) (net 42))
 (segment (start 203.10856 74.79538) (end 201.35856 74.79538) (width 0.25) (layer F.Cu) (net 42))
 (segment (start 198.619059 74.7903) (end 196.66712 76.742239) (width 0.25) (layer F.Cu) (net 42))
 (segment (start 196.66712 76.742239) (end 197.73392 76.742239) (width 0.25) (layer F.Cu) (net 42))
 (segment (start 201.35348 74.7903) (end 198.619059 74.7903) (width 0.25) (layer F.Cu) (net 42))
 (via (at 185.1 75.5) (size 0.8) (drill 0.4) (layers F.Cu B.Cu) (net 42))
 (segment (start 184.4 74.8) (end 185.1 75.5) (width 0.25) (layer B.Cu) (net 42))
 (segment (start 179 74.8) (end 184.4 74.8) (width 0.25) (layer B.Cu) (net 42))
 (segment (start 186.907924 76.742239) (end 196.66712 76.742239) (width 0.25) (layer F.Cu) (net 42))
 (segment (start 185.665685 75.5) (end 186.907924 76.742239) (width 0.25) (layer F.Cu) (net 42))
 (segment (start 185.1 75.5) (end 185.665685 75.5) (width 0.25) (layer F.Cu) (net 42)))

